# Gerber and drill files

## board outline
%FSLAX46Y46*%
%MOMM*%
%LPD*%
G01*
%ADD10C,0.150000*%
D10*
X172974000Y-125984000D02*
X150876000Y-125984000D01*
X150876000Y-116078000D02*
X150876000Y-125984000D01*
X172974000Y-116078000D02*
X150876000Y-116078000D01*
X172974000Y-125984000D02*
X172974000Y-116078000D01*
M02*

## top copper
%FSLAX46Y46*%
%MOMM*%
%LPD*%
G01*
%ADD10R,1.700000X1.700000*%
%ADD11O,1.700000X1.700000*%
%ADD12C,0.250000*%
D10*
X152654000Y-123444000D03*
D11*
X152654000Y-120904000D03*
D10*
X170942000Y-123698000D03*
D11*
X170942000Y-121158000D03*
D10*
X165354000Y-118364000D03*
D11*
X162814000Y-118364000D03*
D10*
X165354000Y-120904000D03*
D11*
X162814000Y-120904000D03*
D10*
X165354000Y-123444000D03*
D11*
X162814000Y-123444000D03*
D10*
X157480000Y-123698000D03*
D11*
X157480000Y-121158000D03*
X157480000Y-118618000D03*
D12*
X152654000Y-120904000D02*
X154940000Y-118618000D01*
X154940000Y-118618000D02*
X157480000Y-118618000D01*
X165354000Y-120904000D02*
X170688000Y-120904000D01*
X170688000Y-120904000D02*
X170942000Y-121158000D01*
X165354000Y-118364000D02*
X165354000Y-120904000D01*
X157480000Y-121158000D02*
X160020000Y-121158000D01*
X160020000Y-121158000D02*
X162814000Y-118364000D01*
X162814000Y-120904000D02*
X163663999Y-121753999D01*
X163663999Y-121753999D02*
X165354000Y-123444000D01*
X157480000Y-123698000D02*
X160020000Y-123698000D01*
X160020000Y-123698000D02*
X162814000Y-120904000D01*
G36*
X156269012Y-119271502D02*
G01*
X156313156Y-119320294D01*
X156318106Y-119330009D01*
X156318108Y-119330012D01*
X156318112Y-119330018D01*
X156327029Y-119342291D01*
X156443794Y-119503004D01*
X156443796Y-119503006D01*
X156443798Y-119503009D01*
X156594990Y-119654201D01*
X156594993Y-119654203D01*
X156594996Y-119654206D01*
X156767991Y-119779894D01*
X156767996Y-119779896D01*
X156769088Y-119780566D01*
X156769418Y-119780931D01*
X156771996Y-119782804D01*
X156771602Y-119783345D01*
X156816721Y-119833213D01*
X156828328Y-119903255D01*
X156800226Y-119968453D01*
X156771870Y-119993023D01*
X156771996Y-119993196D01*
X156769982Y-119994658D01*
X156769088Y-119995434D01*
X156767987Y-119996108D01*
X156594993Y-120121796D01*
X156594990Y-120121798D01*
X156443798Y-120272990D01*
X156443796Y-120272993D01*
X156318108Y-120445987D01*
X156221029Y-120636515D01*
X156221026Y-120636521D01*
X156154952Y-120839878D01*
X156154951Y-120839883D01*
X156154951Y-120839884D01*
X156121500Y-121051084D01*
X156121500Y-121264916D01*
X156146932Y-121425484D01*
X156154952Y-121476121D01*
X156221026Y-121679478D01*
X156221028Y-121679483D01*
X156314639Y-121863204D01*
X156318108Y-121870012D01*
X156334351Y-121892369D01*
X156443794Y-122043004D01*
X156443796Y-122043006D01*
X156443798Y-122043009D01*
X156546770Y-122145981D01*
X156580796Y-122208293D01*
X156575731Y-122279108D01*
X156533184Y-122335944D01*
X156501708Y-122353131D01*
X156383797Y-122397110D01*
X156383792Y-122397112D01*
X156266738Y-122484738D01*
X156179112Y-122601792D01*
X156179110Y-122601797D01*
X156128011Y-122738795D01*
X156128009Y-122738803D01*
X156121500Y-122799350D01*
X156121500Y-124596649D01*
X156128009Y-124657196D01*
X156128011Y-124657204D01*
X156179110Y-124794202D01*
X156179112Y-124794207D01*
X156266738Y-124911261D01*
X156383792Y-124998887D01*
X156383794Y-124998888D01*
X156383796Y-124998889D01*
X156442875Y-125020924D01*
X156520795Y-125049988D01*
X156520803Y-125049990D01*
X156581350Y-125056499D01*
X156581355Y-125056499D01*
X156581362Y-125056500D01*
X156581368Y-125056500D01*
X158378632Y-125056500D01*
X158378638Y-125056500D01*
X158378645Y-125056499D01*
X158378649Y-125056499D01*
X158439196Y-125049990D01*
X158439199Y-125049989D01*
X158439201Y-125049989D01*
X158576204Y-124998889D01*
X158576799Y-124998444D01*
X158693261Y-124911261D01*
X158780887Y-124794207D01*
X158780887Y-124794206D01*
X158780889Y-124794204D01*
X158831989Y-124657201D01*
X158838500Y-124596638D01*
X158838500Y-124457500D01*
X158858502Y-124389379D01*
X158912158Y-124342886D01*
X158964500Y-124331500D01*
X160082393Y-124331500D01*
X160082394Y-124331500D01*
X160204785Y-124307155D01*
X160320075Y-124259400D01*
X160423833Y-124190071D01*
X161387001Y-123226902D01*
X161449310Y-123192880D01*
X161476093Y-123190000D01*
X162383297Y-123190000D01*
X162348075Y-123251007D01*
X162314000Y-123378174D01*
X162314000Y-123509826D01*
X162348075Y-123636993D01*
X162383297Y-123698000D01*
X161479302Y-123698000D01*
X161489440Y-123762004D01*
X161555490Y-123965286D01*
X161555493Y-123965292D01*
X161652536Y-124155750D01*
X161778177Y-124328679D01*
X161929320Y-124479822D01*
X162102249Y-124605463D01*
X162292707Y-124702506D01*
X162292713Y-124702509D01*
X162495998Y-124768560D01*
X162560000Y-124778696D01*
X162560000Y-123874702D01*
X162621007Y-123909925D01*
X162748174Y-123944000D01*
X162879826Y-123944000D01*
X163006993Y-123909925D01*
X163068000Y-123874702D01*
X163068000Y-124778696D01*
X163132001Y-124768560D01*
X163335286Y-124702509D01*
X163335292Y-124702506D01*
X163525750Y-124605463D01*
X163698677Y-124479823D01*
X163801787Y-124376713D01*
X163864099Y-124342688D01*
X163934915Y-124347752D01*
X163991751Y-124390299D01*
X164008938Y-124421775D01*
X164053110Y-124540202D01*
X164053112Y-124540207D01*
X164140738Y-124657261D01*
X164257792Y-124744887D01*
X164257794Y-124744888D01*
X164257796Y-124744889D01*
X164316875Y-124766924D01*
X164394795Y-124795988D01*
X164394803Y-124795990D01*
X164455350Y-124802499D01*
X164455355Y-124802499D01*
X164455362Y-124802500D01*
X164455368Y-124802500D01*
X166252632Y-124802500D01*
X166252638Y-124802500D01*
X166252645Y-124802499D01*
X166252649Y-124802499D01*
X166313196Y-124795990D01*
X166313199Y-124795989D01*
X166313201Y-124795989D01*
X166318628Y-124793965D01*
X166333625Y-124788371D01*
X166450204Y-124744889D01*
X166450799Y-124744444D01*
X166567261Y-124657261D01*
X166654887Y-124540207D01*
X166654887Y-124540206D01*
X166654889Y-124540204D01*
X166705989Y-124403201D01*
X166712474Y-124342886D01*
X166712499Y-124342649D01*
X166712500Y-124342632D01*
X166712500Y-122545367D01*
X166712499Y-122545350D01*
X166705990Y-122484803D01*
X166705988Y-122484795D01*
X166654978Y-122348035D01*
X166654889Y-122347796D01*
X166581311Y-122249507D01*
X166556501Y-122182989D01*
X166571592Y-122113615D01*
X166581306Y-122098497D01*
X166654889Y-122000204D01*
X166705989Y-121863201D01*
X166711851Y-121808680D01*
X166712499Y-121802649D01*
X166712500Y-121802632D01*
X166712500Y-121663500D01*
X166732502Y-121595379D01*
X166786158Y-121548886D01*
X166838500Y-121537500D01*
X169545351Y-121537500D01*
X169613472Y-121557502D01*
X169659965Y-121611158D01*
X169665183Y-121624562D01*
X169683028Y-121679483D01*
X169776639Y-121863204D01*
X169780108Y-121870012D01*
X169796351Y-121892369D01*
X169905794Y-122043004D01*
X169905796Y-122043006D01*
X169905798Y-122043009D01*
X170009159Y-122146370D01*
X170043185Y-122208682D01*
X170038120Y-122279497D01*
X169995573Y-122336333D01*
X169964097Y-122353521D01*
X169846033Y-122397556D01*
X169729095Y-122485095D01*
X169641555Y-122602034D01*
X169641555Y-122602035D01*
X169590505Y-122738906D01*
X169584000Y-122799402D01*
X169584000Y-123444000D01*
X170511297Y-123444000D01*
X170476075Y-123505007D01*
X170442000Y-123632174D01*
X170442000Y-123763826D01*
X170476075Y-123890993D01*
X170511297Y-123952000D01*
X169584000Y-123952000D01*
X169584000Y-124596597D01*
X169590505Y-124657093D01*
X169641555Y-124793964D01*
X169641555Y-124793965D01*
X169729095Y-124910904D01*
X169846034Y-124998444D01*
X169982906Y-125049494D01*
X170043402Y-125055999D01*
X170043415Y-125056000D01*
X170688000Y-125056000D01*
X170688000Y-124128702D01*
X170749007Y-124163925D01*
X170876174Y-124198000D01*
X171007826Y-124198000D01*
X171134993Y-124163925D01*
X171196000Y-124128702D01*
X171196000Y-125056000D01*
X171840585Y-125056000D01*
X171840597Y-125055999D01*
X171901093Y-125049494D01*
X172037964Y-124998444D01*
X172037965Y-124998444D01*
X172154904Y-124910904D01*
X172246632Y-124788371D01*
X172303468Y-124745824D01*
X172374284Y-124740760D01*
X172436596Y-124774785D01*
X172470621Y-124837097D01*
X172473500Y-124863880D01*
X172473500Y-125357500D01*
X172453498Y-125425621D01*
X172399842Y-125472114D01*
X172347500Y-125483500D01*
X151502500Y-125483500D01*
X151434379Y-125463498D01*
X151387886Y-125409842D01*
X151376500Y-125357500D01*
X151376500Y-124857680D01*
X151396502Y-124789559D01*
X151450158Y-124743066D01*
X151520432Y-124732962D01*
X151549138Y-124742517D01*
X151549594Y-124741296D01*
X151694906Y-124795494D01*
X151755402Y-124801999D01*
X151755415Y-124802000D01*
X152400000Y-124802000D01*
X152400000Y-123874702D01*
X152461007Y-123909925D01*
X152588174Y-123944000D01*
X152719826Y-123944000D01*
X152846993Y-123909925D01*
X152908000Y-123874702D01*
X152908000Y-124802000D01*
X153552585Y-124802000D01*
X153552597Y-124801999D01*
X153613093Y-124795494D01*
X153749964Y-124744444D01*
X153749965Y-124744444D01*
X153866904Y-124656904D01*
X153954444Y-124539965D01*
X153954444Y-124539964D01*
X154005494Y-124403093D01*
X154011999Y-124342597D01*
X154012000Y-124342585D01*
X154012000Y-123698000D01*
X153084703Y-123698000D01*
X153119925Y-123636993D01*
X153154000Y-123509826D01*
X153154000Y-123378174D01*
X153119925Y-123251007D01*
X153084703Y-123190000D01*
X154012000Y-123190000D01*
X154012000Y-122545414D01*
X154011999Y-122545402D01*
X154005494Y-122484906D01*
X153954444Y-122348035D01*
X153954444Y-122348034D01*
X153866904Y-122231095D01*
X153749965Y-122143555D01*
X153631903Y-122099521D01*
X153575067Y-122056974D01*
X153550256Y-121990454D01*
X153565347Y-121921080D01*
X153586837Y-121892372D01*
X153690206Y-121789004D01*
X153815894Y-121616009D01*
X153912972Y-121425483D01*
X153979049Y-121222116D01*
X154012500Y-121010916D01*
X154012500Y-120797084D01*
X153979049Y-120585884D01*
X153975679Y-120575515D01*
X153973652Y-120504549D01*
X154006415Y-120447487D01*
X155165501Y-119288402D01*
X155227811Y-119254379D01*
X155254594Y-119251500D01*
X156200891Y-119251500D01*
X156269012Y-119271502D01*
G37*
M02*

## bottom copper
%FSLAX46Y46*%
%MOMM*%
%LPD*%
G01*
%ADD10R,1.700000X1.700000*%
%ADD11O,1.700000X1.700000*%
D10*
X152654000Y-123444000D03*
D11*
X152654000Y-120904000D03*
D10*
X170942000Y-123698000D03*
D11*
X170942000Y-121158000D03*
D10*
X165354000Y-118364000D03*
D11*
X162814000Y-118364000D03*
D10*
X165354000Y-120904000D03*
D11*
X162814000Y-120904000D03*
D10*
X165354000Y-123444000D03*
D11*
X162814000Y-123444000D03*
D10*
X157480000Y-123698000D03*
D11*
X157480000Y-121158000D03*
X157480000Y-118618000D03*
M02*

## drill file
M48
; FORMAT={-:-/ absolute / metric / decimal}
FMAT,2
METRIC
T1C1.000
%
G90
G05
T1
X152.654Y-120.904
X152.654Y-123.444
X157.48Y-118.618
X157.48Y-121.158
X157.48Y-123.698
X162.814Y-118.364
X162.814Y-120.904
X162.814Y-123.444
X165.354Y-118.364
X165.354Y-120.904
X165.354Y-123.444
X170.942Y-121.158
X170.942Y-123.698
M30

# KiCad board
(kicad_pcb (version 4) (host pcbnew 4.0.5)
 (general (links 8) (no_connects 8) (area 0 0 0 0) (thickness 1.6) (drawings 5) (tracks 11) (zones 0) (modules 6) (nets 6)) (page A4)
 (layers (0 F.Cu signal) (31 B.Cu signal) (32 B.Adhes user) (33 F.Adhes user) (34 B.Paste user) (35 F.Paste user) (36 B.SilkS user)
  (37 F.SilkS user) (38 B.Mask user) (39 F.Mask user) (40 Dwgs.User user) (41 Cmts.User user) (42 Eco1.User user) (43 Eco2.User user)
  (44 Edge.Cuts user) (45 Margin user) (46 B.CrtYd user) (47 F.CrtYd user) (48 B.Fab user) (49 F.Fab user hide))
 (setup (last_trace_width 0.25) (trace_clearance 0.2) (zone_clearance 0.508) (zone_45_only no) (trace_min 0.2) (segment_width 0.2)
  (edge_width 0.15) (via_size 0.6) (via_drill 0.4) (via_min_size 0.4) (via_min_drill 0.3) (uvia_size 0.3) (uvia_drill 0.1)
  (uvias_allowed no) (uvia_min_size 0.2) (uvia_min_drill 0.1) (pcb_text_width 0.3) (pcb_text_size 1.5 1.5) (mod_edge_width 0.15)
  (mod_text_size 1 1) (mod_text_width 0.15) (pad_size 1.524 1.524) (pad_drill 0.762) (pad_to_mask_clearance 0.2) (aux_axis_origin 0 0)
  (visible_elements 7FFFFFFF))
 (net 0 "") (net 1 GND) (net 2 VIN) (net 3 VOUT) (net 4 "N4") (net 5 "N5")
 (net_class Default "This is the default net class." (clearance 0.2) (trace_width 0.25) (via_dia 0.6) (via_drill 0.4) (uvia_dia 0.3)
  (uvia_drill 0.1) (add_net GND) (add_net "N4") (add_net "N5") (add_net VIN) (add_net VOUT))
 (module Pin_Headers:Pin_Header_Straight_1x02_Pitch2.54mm (layer F.Cu) (at 152.654 123.444 180)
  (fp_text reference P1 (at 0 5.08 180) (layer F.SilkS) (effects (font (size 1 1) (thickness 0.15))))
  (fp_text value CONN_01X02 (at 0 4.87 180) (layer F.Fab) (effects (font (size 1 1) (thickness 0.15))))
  (pad 1 thru_hole rect (at 0 0 180) (size 1.7 1.7) (drill 1) (layers *.Cu *.Mask) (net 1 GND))
  (pad 2 thru_hole oval (at 0 2.54 180) (size 1.7 1.7) (drill 1) (layers *.Cu *.Mask) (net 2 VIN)))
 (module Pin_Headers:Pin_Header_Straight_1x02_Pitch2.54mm (layer F.Cu) (at 170.942 123.698 180)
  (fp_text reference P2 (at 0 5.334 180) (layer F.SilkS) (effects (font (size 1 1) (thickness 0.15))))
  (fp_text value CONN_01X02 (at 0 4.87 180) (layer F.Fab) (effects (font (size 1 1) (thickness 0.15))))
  (pad 1 thru_hole rect (at 0 0 180) (size 1.7 1.7) (drill 1) (layers *.Cu *.Mask) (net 1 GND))
  (pad 2 thru_hole oval (at 0 2.54 180) (size 1.7 1.7) (drill 1) (layers *.Cu *.Mask) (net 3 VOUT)))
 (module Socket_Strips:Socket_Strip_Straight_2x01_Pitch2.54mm (layer F.Cu) (at 165.354 118.364)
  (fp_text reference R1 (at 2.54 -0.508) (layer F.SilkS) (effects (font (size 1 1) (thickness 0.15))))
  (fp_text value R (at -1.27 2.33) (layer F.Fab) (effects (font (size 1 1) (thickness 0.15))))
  (pad 1 thru_hole rect (at 0 0) (size 1.7 1.7) (drill 1) (layers *.Cu *.Mask) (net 3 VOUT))
  (pad 2 thru_hole oval (at -2.54 0) (size 1.7 1.7) (drill 1) (layers *.Cu *.Mask) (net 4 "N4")))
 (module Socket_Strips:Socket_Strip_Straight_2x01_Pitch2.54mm (layer F.Cu) (at 165.354 120.904)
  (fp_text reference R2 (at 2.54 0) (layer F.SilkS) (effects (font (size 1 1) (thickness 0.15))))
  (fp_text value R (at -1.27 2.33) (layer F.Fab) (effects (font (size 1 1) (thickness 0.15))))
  (pad 1 thru_hole rect (at 0 0) (size 1.7 1.7) (drill 1) (layers *.Cu *.Mask) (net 3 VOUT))
  (pad 2 thru_hole oval (at -2.54 0) (size 1.7 1.7) (drill 1) (layers *.Cu *.Mask) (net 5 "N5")))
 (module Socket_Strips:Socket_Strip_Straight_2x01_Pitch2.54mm (layer F.Cu) (at 165.354 123.444)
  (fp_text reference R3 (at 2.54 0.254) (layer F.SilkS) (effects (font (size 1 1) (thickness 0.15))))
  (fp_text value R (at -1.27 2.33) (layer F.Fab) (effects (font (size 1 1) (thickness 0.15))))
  (pad 1 thru_hole rect (at 0 0) (size 1.7 1.7) (drill 1) (layers *.Cu *.Mask) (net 5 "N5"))
  (pad 2 thru_hole oval (at -2.54 0) (size 1.7 1.7) (drill 1) (layers *.Cu *.Mask) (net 1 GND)))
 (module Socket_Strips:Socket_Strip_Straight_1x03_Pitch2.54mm (layer F.Cu) (at 157.48 123.698 180)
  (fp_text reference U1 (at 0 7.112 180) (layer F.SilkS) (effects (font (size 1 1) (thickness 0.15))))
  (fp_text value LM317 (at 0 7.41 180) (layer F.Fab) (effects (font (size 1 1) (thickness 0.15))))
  (pad 1 thru_hole rect (at 0 0 180) (size 1.7 1.7) (drill 1) (layers *.Cu *.Mask) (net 5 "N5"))
  (pad 2 thru_hole oval (at 0 2.54 180) (size 1.7 1.7) (drill 1) (layers *.Cu *.Mask) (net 4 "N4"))
  (pad 3 thru_hole oval (at 0 5.08 180) (size 1.7 1.7) (drill 1) (layers *.Cu *.Mask) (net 2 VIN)))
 (gr_line (start 172.974 125.984) (end 150.876 125.984) (angle 90) (layer Edge.Cuts) (width 0.15))
 (gr_line (start 150.876 116.078) (end 150.876 125.984) (angle 90) (layer Edge.Cuts) (width 0.15))
 (gr_line (start 172.974 116.078) (end 150.876 116.078) (angle 90) (layer Edge.Cuts) (width 0.15))
 (gr_line (start 172.974 125.984) (end 172.974 116.078) (angle 90) (layer Edge.Cuts) (width 0.15))
 (segment (start 152.654 120.904) (end 154.94 118.618) (width 0.25) (layer F.Cu) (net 2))
 (segment (start 154.94 118.618) (end 157.48 118.618) (width 0.25) (layer F.Cu) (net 2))
 (segment (start 165.354 120.904) (end 170.688 120.904) (width 0.25) (layer F.Cu) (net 3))
 (segment (start 170.688 120.904) (end 170.942 121.158) (width 0.25) (layer F.Cu) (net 3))
 (segment (start 165.354 118.364) (end 165.354 120.904) (width 0.25) (layer F.Cu) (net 3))
 (segment (start 157.48 121.158) (end 160.02 121.158) (width 0.25) (layer F.Cu) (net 4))
 (segment (start 160.02 121.158) (end 162.814 118.364) (width 0.25) (layer F.Cu) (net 4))
 (segment (start 162.814 120.904) (end 163.663999 121.753999) (width 0.25) (layer F.Cu) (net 5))
 (segment (start 163.663999 121.753999) (end 165.354 123.444) (width 0.25) (layer F.Cu) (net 5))
 (segment (start 157.48 123.698) (end 160.02 123.698) (width 0.25) (layer F.Cu) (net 5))
 (segment (start 160.02 123.698) (end 162.814 120.904) (width 0.25) (layer F.Cu) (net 5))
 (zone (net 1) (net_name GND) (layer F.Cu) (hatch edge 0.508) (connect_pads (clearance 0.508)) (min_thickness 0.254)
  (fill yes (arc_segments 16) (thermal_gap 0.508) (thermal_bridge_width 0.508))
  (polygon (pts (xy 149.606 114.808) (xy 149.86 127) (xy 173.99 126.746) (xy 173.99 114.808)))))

